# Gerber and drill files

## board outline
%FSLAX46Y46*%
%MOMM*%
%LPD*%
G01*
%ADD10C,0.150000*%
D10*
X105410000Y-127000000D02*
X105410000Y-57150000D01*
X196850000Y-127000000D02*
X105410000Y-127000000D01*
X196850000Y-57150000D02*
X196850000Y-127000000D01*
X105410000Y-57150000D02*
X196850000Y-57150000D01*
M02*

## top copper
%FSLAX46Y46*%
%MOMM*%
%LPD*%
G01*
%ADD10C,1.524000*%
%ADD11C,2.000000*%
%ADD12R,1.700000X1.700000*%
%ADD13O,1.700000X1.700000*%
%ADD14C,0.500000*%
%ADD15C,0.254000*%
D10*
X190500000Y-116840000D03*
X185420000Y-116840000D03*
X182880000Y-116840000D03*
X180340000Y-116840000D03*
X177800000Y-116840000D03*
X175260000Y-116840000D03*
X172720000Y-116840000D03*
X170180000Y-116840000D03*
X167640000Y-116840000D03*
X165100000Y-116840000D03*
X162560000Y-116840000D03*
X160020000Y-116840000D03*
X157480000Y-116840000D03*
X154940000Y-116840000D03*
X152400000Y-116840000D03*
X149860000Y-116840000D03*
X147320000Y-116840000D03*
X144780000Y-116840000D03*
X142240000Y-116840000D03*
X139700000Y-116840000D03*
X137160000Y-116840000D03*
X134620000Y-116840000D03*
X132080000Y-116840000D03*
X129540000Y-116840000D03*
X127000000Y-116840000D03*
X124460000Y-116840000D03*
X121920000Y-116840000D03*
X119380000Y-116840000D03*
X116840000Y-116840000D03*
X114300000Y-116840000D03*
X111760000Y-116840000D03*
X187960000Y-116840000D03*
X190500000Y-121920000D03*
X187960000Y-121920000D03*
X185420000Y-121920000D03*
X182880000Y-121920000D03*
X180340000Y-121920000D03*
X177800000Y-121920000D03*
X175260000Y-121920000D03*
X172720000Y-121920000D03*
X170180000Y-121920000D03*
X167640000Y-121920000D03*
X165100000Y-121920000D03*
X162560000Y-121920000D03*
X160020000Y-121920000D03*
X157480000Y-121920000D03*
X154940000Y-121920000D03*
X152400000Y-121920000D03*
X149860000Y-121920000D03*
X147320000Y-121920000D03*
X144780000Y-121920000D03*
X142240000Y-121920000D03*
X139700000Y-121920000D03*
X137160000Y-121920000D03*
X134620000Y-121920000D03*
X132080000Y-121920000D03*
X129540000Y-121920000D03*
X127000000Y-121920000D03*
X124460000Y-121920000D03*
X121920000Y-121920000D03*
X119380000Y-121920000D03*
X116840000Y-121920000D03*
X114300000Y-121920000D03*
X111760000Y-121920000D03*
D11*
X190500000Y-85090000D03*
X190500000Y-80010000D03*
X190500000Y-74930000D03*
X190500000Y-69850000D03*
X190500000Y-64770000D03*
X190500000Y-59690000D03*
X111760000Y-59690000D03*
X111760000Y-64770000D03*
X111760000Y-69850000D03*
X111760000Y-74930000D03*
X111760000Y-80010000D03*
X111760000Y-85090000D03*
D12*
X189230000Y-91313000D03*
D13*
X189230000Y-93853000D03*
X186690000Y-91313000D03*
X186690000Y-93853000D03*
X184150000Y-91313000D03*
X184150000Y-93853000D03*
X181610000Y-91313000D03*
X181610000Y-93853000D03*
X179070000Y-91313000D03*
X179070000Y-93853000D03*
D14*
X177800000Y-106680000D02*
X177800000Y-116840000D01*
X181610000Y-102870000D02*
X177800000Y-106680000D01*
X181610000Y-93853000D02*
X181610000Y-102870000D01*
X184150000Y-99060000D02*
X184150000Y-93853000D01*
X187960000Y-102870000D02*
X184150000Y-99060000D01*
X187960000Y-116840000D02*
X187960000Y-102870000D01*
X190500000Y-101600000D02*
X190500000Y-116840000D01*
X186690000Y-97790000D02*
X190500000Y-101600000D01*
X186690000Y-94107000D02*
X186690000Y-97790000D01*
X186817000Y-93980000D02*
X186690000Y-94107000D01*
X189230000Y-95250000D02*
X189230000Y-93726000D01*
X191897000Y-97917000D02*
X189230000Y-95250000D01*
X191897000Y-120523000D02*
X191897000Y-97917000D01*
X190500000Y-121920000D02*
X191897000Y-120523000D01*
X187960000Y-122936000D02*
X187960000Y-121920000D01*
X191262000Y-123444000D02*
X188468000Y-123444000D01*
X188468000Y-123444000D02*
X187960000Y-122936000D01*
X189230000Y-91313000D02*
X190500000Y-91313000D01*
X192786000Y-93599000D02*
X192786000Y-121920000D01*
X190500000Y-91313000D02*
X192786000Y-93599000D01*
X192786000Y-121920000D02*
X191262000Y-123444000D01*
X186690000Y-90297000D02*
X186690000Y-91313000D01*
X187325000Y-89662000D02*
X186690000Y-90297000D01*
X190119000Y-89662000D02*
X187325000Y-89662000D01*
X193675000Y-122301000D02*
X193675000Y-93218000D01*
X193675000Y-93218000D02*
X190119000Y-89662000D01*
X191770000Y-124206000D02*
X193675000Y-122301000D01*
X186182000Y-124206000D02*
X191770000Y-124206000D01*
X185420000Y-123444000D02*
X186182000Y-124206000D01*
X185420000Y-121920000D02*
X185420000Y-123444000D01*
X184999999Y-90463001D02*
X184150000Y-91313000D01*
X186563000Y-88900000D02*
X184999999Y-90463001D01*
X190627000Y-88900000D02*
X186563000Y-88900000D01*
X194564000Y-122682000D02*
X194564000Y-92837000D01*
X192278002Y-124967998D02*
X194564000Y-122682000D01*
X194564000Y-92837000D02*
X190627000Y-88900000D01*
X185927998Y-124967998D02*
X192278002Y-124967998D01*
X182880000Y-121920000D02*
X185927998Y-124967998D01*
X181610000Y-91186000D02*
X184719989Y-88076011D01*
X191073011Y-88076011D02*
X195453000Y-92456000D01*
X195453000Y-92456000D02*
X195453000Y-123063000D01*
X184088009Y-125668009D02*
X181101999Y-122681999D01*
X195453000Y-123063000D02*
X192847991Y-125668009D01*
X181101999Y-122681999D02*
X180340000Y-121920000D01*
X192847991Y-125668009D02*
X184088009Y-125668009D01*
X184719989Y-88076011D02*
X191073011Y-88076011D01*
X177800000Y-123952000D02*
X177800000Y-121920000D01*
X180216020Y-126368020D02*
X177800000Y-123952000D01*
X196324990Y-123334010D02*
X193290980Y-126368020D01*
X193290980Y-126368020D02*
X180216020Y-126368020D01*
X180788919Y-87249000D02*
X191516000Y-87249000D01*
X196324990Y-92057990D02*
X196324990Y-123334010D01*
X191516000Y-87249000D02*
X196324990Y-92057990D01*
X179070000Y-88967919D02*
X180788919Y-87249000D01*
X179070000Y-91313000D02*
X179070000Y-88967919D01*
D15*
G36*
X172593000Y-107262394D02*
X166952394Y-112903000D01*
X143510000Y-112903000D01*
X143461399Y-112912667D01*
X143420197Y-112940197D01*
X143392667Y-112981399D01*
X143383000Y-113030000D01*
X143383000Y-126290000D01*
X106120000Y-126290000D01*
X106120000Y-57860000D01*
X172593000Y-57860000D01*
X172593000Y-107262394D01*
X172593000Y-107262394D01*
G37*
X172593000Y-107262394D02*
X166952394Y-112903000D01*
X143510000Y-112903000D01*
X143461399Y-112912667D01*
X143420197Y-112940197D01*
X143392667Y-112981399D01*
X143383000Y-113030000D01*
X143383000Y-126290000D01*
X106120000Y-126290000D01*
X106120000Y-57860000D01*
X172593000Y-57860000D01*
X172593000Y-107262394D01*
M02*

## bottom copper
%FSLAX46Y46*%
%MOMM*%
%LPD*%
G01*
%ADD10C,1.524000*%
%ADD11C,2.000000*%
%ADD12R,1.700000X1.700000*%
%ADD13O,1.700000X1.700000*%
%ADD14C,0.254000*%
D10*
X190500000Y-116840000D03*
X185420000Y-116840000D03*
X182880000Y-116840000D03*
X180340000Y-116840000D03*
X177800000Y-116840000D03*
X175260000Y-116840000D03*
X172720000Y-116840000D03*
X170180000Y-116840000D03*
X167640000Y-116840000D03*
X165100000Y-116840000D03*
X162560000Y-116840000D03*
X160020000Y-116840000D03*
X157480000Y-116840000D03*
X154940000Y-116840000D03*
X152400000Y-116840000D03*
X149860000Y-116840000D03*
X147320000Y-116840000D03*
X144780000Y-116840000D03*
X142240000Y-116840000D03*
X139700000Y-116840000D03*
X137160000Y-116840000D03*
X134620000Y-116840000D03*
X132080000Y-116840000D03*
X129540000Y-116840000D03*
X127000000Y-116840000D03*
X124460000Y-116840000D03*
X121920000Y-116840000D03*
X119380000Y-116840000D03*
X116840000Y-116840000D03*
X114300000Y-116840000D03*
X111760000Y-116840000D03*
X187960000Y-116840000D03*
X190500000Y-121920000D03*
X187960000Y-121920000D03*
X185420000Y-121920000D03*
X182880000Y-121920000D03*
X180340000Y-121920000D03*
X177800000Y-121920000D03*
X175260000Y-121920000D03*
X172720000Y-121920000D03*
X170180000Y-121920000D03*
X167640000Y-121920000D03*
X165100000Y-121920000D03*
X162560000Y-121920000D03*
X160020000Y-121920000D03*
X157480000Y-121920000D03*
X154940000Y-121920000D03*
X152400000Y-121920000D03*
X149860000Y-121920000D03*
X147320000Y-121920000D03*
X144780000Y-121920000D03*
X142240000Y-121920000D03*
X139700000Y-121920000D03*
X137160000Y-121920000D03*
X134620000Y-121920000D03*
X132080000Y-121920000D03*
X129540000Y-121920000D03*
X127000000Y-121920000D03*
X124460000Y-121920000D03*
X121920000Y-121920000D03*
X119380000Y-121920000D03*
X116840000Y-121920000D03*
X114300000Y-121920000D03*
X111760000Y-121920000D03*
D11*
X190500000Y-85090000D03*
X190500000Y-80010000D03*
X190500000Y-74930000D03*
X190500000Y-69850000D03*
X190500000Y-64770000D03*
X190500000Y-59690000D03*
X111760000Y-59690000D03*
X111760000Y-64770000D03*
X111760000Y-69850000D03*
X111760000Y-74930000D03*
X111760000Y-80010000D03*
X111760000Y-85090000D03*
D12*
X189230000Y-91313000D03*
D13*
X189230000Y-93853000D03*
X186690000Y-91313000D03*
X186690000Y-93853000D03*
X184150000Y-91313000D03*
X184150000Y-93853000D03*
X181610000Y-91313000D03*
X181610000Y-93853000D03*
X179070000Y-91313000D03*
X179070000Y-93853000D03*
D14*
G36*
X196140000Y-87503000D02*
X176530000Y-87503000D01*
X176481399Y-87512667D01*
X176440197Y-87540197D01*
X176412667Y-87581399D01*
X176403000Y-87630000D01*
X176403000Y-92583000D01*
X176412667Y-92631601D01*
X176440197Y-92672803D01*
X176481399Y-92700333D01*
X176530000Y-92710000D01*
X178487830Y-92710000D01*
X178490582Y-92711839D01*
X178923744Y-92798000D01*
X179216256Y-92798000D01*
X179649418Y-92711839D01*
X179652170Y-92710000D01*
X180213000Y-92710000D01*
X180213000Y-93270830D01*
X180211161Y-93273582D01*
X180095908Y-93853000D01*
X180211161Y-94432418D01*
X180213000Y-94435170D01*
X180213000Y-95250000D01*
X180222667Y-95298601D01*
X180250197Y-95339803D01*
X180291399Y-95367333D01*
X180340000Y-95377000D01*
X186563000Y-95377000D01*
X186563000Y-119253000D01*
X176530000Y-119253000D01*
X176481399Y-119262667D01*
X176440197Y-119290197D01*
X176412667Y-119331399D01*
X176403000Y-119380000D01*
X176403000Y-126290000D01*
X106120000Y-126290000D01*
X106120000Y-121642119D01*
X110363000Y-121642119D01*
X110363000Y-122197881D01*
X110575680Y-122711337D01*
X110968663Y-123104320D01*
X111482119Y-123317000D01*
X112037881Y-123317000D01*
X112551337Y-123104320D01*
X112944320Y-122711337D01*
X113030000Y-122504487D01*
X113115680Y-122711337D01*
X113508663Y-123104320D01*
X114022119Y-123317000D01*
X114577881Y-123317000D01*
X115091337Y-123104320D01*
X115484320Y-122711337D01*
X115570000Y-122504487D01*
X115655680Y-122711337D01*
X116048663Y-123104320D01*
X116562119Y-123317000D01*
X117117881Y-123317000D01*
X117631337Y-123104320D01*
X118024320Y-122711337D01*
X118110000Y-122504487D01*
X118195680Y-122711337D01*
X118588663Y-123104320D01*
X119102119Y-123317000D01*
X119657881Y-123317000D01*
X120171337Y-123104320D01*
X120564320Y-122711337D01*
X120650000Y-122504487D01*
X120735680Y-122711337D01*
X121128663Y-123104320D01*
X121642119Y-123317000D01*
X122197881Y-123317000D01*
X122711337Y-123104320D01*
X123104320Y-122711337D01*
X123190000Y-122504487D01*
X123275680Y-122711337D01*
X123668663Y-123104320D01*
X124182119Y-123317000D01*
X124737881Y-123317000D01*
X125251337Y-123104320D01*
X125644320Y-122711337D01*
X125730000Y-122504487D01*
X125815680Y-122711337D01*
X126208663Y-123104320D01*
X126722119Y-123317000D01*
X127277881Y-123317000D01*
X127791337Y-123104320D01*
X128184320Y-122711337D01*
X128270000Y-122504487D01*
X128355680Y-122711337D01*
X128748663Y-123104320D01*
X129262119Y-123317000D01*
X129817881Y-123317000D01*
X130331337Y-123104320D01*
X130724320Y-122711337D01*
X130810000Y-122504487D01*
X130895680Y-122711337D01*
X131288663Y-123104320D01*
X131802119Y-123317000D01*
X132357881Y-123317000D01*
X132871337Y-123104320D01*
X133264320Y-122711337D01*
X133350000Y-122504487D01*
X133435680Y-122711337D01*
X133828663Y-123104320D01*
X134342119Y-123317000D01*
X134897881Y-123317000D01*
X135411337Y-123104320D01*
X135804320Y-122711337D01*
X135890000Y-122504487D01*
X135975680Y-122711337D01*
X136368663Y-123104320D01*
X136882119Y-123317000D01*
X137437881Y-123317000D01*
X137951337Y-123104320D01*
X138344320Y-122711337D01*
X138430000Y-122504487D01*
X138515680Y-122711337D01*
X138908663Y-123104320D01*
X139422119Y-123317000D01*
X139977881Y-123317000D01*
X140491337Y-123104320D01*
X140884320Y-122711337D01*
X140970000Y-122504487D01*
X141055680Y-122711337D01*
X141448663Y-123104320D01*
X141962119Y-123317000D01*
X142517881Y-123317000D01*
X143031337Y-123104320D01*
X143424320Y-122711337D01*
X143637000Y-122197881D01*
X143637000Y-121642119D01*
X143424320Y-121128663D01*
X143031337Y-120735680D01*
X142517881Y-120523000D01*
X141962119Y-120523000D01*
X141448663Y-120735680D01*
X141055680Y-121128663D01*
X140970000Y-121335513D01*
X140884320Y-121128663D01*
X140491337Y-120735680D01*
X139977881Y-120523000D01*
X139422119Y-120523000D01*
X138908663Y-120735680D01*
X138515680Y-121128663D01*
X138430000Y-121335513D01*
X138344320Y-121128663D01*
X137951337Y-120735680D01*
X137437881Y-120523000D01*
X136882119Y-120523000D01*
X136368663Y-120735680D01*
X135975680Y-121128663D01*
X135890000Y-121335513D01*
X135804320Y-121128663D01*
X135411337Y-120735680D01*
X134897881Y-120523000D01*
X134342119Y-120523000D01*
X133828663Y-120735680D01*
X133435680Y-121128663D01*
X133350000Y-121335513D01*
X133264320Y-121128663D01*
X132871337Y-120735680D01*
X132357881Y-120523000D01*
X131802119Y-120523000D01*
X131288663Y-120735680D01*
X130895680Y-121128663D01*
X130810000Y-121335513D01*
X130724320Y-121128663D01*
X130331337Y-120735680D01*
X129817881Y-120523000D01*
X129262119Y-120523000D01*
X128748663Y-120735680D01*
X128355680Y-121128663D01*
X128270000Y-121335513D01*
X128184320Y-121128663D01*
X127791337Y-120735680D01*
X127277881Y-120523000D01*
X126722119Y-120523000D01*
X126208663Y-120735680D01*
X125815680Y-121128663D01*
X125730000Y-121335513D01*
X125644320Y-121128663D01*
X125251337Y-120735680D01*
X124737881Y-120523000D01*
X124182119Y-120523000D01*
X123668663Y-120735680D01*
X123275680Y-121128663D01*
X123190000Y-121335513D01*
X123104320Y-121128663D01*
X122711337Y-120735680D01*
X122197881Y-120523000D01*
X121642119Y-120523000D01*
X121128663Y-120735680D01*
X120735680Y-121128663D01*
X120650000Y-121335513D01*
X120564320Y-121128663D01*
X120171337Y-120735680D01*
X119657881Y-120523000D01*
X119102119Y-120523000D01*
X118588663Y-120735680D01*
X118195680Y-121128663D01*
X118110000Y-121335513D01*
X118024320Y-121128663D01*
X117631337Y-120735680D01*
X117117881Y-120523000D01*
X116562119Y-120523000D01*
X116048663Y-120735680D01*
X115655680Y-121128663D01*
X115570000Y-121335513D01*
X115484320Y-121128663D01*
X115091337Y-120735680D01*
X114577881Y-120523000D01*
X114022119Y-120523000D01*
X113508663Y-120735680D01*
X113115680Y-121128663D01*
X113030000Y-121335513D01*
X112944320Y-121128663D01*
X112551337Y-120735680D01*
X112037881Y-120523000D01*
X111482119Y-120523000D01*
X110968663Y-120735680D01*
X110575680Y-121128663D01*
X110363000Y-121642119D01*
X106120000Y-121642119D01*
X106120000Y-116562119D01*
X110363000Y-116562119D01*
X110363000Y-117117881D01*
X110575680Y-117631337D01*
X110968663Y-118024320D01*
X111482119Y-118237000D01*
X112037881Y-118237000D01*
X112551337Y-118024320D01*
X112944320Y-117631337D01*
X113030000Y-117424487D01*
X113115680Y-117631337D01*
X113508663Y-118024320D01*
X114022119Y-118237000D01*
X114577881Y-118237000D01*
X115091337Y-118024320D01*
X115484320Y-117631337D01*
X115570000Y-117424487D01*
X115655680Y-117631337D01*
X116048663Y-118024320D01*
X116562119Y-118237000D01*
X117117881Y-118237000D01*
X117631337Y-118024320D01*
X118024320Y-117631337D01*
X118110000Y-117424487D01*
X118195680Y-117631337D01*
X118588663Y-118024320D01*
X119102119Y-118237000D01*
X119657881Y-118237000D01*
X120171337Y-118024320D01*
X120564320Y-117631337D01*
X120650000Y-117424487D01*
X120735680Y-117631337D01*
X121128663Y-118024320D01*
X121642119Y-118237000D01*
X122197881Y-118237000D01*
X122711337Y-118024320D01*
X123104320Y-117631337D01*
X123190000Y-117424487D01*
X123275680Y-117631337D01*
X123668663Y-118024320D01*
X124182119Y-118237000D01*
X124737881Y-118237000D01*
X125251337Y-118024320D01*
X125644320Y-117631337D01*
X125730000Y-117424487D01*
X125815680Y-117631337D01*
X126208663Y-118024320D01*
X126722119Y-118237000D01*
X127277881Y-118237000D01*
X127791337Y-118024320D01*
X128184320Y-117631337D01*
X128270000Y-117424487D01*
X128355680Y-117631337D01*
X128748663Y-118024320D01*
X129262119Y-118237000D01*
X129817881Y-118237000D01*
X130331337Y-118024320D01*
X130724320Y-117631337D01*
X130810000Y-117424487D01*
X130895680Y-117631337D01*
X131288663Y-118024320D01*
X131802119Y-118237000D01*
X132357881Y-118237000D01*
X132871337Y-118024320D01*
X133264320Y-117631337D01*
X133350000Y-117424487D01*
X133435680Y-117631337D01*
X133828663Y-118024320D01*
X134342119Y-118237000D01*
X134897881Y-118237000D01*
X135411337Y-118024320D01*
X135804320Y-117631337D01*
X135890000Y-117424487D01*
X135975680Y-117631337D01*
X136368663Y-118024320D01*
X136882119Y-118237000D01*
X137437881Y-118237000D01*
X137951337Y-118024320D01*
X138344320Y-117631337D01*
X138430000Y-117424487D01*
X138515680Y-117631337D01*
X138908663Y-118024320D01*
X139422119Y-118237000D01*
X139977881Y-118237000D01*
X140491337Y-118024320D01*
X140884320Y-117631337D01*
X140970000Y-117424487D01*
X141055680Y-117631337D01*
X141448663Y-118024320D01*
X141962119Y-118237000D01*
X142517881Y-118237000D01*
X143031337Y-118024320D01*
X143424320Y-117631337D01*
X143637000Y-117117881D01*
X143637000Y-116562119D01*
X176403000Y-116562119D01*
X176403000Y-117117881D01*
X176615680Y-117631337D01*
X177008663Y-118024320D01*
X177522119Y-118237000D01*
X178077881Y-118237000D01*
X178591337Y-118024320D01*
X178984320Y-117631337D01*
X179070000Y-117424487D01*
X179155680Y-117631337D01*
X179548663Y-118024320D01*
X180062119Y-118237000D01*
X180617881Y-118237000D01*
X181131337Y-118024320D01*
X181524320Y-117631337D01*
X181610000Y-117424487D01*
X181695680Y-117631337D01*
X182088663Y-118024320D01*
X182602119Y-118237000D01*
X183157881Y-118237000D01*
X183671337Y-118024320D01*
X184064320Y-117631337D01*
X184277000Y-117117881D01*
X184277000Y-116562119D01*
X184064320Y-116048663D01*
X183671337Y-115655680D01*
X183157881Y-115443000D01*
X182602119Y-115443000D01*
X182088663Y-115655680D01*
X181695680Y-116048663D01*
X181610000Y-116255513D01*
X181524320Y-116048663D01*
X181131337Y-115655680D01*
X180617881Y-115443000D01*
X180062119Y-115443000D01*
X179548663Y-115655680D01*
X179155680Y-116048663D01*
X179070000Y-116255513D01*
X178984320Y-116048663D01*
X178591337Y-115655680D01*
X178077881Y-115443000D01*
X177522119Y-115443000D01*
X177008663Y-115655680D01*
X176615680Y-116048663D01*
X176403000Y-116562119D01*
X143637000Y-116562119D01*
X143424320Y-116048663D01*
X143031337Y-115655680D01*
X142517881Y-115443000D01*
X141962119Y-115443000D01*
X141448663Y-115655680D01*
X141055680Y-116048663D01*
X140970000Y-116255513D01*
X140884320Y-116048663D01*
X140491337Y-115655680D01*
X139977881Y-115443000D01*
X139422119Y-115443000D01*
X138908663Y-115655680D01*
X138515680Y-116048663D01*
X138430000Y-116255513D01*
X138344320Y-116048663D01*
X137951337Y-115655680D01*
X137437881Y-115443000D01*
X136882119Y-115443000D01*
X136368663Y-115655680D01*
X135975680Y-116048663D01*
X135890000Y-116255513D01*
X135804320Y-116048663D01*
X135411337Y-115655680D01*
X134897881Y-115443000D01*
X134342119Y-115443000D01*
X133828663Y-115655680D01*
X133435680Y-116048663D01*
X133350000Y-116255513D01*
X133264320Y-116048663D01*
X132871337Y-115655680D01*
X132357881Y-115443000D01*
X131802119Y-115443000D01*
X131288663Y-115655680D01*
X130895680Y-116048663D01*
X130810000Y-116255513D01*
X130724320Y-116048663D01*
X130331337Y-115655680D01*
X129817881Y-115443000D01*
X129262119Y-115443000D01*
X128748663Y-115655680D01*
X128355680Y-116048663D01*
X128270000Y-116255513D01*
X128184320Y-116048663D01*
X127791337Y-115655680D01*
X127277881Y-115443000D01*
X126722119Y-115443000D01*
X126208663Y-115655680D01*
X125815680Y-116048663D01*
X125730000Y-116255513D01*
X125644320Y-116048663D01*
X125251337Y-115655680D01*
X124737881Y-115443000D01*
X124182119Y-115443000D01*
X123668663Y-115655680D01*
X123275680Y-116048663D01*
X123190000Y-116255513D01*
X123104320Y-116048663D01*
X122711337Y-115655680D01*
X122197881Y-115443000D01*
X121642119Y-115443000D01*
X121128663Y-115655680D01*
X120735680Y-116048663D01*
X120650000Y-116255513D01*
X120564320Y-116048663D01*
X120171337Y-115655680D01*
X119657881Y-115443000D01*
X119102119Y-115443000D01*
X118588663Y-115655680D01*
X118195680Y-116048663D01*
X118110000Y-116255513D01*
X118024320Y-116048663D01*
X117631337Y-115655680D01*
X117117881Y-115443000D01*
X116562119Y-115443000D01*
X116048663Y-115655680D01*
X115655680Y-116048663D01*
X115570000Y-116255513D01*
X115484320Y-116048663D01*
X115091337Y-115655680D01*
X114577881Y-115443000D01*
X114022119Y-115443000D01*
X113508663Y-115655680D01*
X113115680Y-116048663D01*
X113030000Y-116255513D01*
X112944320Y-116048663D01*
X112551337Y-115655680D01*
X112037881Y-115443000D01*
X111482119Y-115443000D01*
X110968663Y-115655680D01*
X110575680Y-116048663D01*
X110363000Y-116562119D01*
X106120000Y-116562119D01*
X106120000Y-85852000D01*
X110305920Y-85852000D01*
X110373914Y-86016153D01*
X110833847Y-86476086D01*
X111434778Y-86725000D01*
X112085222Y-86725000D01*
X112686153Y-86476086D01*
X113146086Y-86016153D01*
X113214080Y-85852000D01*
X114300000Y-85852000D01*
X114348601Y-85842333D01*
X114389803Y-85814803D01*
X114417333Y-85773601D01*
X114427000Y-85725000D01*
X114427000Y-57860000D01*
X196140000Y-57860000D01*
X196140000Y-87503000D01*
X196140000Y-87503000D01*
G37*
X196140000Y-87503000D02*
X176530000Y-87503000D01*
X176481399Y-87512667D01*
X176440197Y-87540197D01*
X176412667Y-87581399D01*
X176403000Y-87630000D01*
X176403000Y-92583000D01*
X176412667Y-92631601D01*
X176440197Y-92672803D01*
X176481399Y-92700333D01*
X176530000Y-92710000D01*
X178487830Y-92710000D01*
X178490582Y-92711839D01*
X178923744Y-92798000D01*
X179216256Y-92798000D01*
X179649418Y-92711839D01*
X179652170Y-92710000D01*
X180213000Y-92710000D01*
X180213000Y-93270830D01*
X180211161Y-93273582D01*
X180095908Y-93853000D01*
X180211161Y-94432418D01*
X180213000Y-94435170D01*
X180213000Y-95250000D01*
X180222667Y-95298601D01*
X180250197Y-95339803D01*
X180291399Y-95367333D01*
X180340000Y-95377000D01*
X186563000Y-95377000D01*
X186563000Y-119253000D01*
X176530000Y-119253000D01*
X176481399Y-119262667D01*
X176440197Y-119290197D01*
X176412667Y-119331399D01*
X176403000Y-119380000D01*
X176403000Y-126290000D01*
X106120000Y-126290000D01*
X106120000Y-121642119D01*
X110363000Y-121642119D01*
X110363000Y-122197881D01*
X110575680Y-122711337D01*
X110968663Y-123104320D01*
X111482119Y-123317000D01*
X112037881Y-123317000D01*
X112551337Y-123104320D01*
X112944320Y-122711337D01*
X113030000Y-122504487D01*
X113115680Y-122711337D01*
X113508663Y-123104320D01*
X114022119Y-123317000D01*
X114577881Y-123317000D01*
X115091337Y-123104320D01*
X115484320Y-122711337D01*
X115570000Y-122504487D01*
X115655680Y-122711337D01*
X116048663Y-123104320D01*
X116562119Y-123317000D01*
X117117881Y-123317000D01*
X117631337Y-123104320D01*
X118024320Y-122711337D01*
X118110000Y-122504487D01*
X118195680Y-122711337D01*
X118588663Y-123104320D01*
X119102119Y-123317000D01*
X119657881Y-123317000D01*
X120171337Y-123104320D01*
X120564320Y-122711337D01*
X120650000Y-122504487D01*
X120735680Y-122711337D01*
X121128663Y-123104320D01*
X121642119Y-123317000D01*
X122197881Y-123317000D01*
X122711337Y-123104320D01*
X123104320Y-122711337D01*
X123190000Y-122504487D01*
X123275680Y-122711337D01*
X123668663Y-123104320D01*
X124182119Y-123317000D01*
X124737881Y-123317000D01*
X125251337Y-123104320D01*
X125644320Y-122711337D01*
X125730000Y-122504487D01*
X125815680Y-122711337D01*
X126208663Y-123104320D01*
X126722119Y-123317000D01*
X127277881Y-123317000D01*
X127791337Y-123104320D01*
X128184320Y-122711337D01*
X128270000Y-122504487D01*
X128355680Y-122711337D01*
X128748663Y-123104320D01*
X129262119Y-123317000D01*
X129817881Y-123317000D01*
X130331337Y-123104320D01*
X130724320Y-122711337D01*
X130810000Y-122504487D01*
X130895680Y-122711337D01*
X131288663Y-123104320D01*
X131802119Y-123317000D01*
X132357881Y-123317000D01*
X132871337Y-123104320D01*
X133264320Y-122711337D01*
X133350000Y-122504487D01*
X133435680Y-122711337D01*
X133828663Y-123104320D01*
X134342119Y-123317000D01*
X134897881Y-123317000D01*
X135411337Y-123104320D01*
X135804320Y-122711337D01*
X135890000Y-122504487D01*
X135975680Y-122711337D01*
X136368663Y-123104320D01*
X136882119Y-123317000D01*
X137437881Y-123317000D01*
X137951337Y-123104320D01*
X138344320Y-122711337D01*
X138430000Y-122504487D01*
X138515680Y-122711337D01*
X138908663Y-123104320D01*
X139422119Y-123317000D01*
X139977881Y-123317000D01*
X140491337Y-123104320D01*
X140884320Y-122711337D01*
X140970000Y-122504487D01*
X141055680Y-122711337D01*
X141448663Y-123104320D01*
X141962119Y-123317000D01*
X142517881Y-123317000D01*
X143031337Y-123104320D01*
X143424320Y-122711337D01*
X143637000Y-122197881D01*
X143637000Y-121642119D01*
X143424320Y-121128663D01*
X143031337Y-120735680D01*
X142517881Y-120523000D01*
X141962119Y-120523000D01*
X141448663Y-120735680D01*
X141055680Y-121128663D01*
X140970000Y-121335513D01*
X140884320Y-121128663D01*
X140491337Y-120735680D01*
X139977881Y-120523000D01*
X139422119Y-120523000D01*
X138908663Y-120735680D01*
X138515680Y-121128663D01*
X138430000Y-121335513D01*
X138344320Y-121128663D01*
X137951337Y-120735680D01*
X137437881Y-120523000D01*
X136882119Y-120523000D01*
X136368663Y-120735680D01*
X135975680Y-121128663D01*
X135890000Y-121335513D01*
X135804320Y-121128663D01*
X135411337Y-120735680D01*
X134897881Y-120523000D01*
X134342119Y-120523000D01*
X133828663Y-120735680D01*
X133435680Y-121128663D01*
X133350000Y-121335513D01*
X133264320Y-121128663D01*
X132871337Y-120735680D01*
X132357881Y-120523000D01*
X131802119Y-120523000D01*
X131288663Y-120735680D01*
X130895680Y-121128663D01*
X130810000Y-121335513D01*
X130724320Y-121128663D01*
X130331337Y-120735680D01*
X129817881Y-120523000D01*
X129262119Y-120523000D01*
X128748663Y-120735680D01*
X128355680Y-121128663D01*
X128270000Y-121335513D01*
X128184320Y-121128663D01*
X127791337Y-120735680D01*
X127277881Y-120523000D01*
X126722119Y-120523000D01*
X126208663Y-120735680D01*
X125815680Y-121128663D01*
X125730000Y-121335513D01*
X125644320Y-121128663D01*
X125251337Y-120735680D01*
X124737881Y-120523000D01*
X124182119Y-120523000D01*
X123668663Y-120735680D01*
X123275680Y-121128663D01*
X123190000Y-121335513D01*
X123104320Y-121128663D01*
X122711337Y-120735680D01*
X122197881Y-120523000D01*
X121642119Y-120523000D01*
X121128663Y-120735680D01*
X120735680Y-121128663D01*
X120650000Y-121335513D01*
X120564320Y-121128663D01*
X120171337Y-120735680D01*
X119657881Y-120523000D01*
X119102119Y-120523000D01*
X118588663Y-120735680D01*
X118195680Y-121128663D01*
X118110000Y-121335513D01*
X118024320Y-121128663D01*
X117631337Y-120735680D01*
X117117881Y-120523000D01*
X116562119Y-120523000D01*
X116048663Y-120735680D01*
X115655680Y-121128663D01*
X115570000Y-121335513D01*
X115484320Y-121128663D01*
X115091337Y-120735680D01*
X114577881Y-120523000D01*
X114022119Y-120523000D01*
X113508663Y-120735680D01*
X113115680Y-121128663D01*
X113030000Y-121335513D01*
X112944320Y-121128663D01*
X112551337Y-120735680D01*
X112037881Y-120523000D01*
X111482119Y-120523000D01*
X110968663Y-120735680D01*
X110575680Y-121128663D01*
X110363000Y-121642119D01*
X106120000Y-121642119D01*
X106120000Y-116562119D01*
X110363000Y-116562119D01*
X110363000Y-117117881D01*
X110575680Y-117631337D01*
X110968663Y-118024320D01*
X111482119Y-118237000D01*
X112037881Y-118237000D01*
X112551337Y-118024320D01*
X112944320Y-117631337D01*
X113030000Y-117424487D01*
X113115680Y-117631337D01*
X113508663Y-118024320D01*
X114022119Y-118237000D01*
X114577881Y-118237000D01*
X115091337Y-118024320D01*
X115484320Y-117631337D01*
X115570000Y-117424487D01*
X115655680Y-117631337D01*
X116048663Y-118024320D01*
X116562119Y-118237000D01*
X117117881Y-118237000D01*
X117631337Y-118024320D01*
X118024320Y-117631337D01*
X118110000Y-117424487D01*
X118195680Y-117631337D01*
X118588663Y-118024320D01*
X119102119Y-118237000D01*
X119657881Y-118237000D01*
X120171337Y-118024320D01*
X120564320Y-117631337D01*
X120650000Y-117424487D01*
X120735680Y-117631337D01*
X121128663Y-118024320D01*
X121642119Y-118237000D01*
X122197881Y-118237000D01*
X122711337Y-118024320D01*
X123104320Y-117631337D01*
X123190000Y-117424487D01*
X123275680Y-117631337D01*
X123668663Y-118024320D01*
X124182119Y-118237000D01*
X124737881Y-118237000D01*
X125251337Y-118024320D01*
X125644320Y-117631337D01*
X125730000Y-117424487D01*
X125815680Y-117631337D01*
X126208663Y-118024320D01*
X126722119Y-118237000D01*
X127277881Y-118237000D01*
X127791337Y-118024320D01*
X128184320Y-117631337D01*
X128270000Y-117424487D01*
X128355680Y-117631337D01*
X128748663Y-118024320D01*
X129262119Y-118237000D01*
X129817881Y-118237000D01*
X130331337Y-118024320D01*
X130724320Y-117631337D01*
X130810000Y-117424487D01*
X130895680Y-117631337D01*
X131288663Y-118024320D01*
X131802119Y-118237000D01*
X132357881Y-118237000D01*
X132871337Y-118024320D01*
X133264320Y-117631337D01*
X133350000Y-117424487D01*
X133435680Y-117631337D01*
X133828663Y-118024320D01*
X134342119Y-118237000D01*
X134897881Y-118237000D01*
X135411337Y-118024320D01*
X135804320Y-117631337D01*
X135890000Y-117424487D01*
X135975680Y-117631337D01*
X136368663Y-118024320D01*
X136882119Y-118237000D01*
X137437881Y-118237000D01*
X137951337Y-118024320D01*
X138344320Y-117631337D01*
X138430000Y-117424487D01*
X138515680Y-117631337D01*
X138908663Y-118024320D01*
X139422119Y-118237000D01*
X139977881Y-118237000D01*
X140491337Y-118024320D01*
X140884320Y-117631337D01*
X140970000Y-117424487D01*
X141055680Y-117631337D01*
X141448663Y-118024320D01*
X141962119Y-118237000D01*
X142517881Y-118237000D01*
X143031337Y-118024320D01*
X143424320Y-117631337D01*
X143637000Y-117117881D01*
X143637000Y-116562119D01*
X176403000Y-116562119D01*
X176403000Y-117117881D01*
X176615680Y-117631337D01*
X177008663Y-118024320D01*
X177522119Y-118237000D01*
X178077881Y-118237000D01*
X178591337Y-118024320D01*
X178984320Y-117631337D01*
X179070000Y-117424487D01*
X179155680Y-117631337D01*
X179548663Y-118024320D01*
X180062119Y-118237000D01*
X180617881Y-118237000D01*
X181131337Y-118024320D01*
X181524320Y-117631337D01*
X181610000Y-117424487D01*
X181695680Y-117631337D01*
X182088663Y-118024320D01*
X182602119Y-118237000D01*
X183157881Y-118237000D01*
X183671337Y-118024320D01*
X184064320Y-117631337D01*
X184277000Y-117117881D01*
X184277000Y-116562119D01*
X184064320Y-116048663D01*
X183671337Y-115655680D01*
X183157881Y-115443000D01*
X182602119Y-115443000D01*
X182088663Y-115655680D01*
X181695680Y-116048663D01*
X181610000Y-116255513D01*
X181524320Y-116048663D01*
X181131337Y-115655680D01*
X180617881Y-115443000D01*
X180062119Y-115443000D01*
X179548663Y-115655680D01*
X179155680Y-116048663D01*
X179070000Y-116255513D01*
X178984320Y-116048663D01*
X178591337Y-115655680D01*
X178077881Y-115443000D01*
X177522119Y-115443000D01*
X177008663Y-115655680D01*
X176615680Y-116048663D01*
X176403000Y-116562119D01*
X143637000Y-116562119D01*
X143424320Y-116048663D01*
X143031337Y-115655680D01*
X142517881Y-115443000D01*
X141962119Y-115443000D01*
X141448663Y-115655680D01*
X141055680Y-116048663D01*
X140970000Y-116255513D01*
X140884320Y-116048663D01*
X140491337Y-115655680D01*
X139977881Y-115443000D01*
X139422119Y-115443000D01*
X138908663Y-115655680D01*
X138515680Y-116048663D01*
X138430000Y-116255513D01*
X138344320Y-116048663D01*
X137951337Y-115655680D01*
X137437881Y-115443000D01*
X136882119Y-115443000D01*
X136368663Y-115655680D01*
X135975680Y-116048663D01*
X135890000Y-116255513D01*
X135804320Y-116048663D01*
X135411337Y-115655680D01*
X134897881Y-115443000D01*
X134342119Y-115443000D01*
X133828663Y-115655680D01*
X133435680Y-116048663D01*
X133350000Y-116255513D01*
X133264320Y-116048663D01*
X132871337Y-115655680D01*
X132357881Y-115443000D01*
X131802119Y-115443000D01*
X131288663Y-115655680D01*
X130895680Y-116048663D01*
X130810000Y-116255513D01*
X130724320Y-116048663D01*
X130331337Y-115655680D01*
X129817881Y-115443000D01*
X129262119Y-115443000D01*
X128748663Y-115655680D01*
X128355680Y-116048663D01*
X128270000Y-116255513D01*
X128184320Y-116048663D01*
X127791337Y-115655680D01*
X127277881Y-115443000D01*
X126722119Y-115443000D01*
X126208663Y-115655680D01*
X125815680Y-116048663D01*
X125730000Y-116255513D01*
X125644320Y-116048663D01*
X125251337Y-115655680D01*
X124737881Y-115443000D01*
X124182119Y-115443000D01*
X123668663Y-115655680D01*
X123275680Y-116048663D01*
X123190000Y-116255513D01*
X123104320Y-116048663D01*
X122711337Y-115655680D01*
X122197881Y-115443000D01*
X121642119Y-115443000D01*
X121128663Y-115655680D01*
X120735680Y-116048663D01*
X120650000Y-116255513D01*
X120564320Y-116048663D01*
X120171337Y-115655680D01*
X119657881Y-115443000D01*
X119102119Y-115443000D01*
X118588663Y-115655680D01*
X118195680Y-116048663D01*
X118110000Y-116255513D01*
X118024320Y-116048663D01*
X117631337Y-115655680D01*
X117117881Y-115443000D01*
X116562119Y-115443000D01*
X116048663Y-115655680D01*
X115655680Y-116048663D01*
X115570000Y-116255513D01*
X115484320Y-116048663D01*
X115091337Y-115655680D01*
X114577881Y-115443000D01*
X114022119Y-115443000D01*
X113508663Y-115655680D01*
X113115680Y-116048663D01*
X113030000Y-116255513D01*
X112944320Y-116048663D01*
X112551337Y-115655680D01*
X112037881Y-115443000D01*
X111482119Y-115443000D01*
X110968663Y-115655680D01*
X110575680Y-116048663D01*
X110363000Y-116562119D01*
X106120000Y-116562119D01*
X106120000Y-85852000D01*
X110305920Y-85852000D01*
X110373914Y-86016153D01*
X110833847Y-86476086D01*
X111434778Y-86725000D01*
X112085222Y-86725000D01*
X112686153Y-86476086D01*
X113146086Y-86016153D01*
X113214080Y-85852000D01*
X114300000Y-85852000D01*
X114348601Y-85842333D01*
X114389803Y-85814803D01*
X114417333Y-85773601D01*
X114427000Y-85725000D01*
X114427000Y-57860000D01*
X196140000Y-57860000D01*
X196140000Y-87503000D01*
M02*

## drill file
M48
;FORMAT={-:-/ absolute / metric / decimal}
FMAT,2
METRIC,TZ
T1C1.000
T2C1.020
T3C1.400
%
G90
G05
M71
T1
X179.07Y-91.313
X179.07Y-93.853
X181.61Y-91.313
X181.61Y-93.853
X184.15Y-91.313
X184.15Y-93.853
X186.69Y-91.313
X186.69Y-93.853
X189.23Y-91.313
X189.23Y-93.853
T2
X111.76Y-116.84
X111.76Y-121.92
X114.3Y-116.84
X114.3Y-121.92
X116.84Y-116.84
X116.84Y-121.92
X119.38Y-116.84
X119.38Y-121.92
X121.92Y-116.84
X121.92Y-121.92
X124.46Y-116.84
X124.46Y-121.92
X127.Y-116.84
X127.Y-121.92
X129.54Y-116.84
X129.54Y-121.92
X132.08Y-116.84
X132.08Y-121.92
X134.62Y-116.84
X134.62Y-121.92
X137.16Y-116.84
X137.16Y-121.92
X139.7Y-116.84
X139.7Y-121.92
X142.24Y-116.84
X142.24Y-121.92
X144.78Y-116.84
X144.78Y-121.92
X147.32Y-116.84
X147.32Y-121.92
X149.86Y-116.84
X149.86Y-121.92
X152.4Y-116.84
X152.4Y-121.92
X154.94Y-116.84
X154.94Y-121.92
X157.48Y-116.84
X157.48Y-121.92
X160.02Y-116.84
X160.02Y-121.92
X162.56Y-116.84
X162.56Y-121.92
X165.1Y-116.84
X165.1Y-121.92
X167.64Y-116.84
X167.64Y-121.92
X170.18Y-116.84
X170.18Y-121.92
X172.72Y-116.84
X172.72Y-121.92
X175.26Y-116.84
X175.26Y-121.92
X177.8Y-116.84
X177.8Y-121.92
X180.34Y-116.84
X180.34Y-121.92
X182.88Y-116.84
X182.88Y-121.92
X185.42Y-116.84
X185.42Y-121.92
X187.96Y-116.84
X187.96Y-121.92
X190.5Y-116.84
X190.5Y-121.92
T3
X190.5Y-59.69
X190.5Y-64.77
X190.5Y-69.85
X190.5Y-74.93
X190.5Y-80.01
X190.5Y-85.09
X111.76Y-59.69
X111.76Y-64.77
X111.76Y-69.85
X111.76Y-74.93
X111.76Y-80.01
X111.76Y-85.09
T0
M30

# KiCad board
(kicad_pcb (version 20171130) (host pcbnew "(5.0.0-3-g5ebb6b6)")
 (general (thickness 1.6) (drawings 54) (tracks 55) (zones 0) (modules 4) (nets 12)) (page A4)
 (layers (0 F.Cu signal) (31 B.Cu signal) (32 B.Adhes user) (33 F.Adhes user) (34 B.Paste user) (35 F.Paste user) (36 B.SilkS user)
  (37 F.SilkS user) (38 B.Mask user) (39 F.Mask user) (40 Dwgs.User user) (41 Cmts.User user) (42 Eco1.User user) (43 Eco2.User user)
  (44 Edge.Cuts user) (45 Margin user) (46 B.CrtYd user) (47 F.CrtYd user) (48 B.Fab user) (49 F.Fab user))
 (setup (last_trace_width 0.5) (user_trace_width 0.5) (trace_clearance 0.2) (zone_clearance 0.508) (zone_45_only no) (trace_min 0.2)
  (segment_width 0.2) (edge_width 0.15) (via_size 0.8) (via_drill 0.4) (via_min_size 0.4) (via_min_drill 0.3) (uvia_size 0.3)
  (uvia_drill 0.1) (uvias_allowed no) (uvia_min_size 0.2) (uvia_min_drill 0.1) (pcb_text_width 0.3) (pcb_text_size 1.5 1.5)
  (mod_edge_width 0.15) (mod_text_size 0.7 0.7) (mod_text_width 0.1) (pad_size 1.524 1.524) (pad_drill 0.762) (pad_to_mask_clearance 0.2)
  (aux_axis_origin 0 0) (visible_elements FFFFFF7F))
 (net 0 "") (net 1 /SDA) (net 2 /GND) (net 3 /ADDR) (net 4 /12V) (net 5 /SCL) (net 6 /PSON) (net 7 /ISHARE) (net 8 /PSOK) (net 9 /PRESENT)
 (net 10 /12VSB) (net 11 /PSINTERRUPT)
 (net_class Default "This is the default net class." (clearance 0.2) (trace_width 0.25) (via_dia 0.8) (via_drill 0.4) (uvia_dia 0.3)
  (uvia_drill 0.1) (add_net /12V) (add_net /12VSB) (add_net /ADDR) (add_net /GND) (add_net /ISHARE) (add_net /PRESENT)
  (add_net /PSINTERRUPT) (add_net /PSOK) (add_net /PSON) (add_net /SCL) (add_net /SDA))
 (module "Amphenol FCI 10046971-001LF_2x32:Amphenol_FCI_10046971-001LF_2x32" (layer B.Cu) (at 151.13 119.38 270)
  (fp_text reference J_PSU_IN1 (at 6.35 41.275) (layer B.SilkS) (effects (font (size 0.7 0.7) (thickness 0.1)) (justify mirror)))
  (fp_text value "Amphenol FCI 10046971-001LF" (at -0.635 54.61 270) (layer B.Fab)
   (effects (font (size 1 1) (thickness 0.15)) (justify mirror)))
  (pad 32 thru_hole circle (at -2.54 -39.37 270) (size 1.524 1.524) (drill 1.02) (layers *.Cu *.Mask) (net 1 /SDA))
  (pad 30 thru_hole circle (at -2.54 -34.29 270) (size 1.524 1.524) (drill 1.02) (layers *.Cu *.Mask) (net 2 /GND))
  (pad 29 thru_hole circle (at -2.54 -31.75 270) (size 1.524 1.524) (drill 1.02) (layers *.Cu *.Mask))
  (pad 28 thru_hole circle (at -2.54 -29.21 270) (size 1.524 1.524) (drill 1.02) (layers *.Cu *.Mask))
  (pad 27 thru_hole circle (at -2.54 -26.67 270) (size 1.524 1.524) (drill 1.02) (layers *.Cu *.Mask) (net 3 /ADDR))
  (pad 26 thru_hole circle (at -2.54 -24.13 270) (size 1.524 1.524) (drill 1.02) (layers *.Cu *.Mask) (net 2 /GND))
  (pad 25 thru_hole circle (at -2.54 -21.59 270) (size 1.524 1.524) (drill 1.02) (layers *.Cu *.Mask) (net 2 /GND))
  (pad 24 thru_hole circle (at -2.54 -19.05 270) (size 1.524 1.524) (drill 1.02) (layers *.Cu *.Mask) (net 2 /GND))
  (pad 23 thru_hole circle (at -2.54 -16.51 270) (size 1.524 1.524) (drill 1.02) (layers *.Cu *.Mask) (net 2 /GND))
  (pad 22 thru_hole circle (at -2.54 -13.97 270) (size 1.524 1.524) (drill 1.02) (layers *.Cu *.Mask) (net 2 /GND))
  (pad 21 thru_hole circle (at -2.54 -11.43 270) (size 1.524 1.524) (drill 1.02) (layers *.Cu *.Mask) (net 2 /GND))
  (pad 20 thru_hole circle (at -2.54 -8.89 270) (size 1.524 1.524) (drill 1.02) (layers *.Cu *.Mask) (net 2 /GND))
  (pad 19 thru_hole circle (at -2.54 -6.35 270) (size 1.524 1.524) (drill 1.02) (layers *.Cu *.Mask) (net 2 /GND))
  (pad 18 thru_hole circle (at -2.54 -3.81 270) (size 1.524 1.524) (drill 1.02) (layers *.Cu *.Mask) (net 2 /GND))
  (pad 17 thru_hole circle (at -2.54 -1.27 270) (size 1.524 1.524) (drill 1.02) (layers *.Cu *.Mask) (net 2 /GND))
  (pad 16 thru_hole circle (at -2.54 1.27 270) (size 1.524 1.524) (drill 1.02) (layers *.Cu *.Mask) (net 2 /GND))
  (pad 15 thru_hole circle (at -2.54 3.81 270) (size 1.524 1.524) (drill 1.02) (layers *.Cu *.Mask) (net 2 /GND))
  (pad 14 thru_hole circle (at -2.54 6.35 270) (size 1.524 1.524) (drill 1.02) (layers *.Cu *.Mask) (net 2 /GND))
  (pad 13 thru_hole circle (at -2.54 8.89 270) (size 1.524 1.524) (drill 1.02) (layers *.Cu *.Mask) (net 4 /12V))
  (pad 12 thru_hole circle (at -2.54 11.43 270) (size 1.524 1.524) (drill 1.02) (layers *.Cu *.Mask) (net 4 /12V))
  (pad 11 thru_hole circle (at -2.54 13.97 270) (size 1.524 1.524) (drill 1.02) (layers *.Cu *.Mask) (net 4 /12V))
  (pad 10 thru_hole circle (at -2.54 16.51 270) (size 1.524 1.524) (drill 1.02) (layers *.Cu *.Mask) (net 4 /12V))
  (pad 9 thru_hole circle (at -2.54 19.05 270) (size 1.524 1.524) (drill 1.02) (layers *.Cu *.Mask) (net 4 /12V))
  (pad 8 thru_hole circle (at -2.54 21.59 270) (size 1.524 1.524) (drill 1.02) (layers *.Cu *.Mask) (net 4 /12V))
  (pad 7 thru_hole circle (at -2.54 24.13 270) (size 1.524 1.524) (drill 1.02) (layers *.Cu *.Mask) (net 4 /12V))
  (pad 6 thru_hole circle (at -2.54 26.67 270) (size 1.524 1.524) (drill 1.02) (layers *.Cu *.Mask) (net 4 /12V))
  (pad 5 thru_hole circle (at -2.54 29.21 270) (size 1.524 1.524) (drill 1.02) (layers *.Cu *.Mask) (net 4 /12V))
  (pad 4 thru_hole circle (at -2.54 31.75 270) (size 1.524 1.524) (drill 1.02) (layers *.Cu *.Mask) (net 4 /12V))
  (pad 3 thru_hole circle (at -2.54 34.29 270) (size 1.524 1.524) (drill 1.02) (layers *.Cu *.Mask) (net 4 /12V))
  (pad 2 thru_hole circle (at -2.54 36.83 270) (size 1.524 1.524) (drill 1.02) (layers *.Cu *.Mask) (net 4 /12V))
  (pad 1 thru_hole circle (at -2.54 39.37 270) (size 1.524 1.524) (drill 1.02) (layers *.Cu *.Mask) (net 4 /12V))
  (pad 31 thru_hole circle (at -2.54 -36.83 270) (size 1.524 1.524) (drill 1.02) (layers *.Cu *.Mask) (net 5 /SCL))
  (pad 33 thru_hole circle (at 2.54 -39.37 270) (size 1.524 1.524) (drill 1.02) (layers *.Cu *.Mask) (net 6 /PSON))
  (pad 34 thru_hole circle (at 2.54 -36.83 270) (size 1.524 1.524) (drill 1.02) (layers *.Cu *.Mask) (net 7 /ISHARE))
  (pad 35 thru_hole circle (at 2.54 -34.29 270) (size 1.524 1.524) (drill 1.02) (layers *.Cu *.Mask) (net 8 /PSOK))
  (pad 36 thru_hole circle (at 2.54 -31.75 270) (size 1.524 1.524) (drill 1.02) (layers *.Cu *.Mask) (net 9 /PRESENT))
  (pad 37 thru_hole circle (at 2.54 -29.21 270) (size 1.524 1.524) (drill 1.02) (layers *.Cu *.Mask) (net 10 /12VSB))
  (pad 38 thru_hole circle (at 2.54 -26.67 270) (size 1.524 1.524) (drill 1.02) (layers *.Cu *.Mask) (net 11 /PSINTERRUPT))
  (pad 39 thru_hole circle (at 2.54 -24.13 270) (size 1.524 1.524) (drill 1.02) (layers *.Cu *.Mask) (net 2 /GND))
  (pad 40 thru_hole circle (at 2.54 -21.59 270) (size 1.524 1.524) (drill 1.02) (layers *.Cu *.Mask) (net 2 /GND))
  (pad 41 thru_hole circle (at 2.54 -19.05 270) (size 1.524 1.524) (drill 1.02) (layers *.Cu *.Mask) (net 2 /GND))
  (pad 42 thru_hole circle (at 2.54 -16.51 270) (size 1.524 1.524) (drill 1.02) (layers *.Cu *.Mask) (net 2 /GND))
  (pad 43 thru_hole circle (at 2.54 -13.97 270) (size 1.524 1.524) (drill 1.02) (layers *.Cu *.Mask) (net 2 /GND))
  (pad 44 thru_hole circle (at 2.54 -11.43 270) (size 1.524 1.524) (drill 1.02) (layers *.Cu *.Mask) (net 2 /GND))
  (pad 45 thru_hole circle (at 2.54 -8.89 270) (size 1.524 1.524) (drill 1.02) (layers *.Cu *.Mask) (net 2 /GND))
  (pad 46 thru_hole circle (at 2.54 -6.35 270) (size 1.524 1.524) (drill 1.02) (layers *.Cu *.Mask) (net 2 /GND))
  (pad 47 thru_hole circle (at 2.54 -3.81 270) (size 1.524 1.524) (drill 1.02) (layers *.Cu *.Mask) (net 2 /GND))
  (pad 48 thru_hole circle (at 2.54 -1.27 270) (size 1.524 1.524) (drill 1.02) (layers *.Cu *.Mask) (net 2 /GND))
  (pad 49 thru_hole circle (at 2.54 1.27 270) (size 1.524 1.524) (drill 1.02) (layers *.Cu *.Mask) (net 2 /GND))
  (pad 50 thru_hole circle (at 2.54 3.81 270) (size 1.524 1.524) (drill 1.02) (layers *.Cu *.Mask) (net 2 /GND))
  (pad 51 thru_hole circle (at 2.54 6.35 270) (size 1.524 1.524) (drill 1.02) (layers *.Cu *.Mask) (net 2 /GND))
  (pad 52 thru_hole circle (at 2.54 8.89 270) (size 1.524 1.524) (drill 1.02) (layers *.Cu *.Mask) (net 4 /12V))
  (pad 53 thru_hole circle (at 2.54 11.43 270) (size 1.524 1.524) (drill 1.02) (layers *.Cu *.Mask) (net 4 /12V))
  (pad 54 thru_hole circle (at 2.54 13.97 270) (size 1.524 1.524) (drill 1.02) (layers *.Cu *.Mask) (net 4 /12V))
  (pad 55 thru_hole circle (at 2.54 16.51 270) (size 1.524 1.524) (drill 1.02) (layers *.Cu *.Mask) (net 4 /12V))
  (pad 56 thru_hole circle (at 2.54 19.05 270) (size 1.524 1.524) (drill 1.02) (layers *.Cu *.Mask) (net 4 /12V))
  (pad 57 thru_hole circle (at 2.54 21.59 270) (size 1.524 1.524) (drill 1.02) (layers *.Cu *.Mask) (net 4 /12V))
  (pad 58 thru_hole circle (at 2.54 24.13 270) (size 1.524 1.524) (drill 1.02) (layers *.Cu *.Mask) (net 4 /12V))
  (pad 59 thru_hole circle (at 2.54 26.67 270) (size 1.524 1.524) (drill 1.02) (layers *.Cu *.Mask) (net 4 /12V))
  (pad 60 thru_hole circle (at 2.54 29.21 270) (size 1.524 1.524) (drill 1.02) (layers *.Cu *.Mask) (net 4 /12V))
  (pad 61 thru_hole circle (at 2.54 31.75 270) (size 1.524 1.524) (drill 1.02) (layers *.Cu *.Mask) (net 4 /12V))
  (pad 62 thru_hole circle (at 2.54 34.29 270) (size 1.524 1.524) (drill 1.02) (layers *.Cu *.Mask) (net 4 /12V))
  (pad 63 thru_hole circle (at 2.54 36.83 270) (size 1.524 1.524) (drill 1.02) (layers *.Cu *.Mask) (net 4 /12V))
  (pad 64 thru_hole circle (at 2.54 39.37 270) (size 1.524 1.524) (drill 1.02) (layers *.Cu *.Mask) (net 4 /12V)))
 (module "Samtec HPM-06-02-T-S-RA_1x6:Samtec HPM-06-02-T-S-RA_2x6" (layer F.Cu) (at 190.5 72.39)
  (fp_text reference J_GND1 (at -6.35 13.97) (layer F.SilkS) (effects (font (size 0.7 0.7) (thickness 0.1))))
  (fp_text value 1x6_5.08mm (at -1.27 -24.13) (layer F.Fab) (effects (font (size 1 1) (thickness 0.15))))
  (pad 6 thru_hole circle (at 0 12.7) (size 2 2) (drill 1.4) (layers *.Cu *.Mask) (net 2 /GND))
  (pad 5 thru_hole circle (at 0 7.62) (size 2 2) (drill 1.4) (layers *.Cu *.Mask) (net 2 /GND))
  (pad 4 thru_hole circle (at 0 2.54) (size 2 2) (drill 1.4) (layers *.Cu *.Mask) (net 2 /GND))
  (pad 3 thru_hole circle (at 0 -2.54) (size 2 2) (drill 1.4) (layers *.Cu *.Mask) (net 2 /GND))
  (pad 2 thru_hole circle (at 0 -7.62) (size 2 2) (drill 1.4) (layers *.Cu *.Mask) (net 2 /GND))
  (pad 1 thru_hole circle (at 0 -12.7) (size 2 2) (drill 1.4) (layers *.Cu *.Mask) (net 2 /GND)))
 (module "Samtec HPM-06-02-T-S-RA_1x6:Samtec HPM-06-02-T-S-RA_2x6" (layer F.Cu) (at 111.76 72.39)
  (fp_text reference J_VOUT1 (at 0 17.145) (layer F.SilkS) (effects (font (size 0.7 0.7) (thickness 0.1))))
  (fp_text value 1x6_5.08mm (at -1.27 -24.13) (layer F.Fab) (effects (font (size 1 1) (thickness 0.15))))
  (pad 1 thru_hole circle (at 0 -12.7) (size 2 2) (drill 1.4) (layers *.Cu *.Mask) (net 4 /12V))
  (pad 2 thru_hole circle (at 0 -7.62) (size 2 2) (drill 1.4) (layers *.Cu *.Mask) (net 4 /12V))
  (pad 3 thru_hole circle (at 0 -2.54) (size 2 2) (drill 1.4) (layers *.Cu *.Mask) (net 4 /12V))
  (pad 4 thru_hole circle (at 0 2.54) (size 2 2) (drill 1.4) (layers *.Cu *.Mask) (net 4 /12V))
  (pad 5 thru_hole circle (at 0 7.62) (size 2 2) (drill 1.4) (layers *.Cu *.Mask) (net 4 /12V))
  (pad 6 thru_hole circle (at 0 12.7) (size 2 2) (drill 1.4) (layers *.Cu *.Mask) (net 4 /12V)))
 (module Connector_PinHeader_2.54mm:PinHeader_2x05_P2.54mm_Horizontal (layer F.Cu) (at 189.23 91.313 270)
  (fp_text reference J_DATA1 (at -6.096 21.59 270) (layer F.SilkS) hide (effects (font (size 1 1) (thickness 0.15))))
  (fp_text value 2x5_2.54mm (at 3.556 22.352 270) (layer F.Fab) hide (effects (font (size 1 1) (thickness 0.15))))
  (pad 1 thru_hole rect (at 0 0 270) (size 1.7 1.7) (drill 1) (layers *.Cu *.Mask) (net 7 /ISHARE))
  (pad 2 thru_hole oval (at 2.54 0 270) (size 1.7 1.7) (drill 1) (layers *.Cu *.Mask) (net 6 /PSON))
  (pad 3 thru_hole oval (at 0 2.54 270) (size 1.7 1.7) (drill 1) (layers *.Cu *.Mask) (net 8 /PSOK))
  (pad 4 thru_hole oval (at 2.54 2.54 270) (size 1.7 1.7) (drill 1) (layers *.Cu *.Mask) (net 1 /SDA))
  (pad 5 thru_hole oval (at 0 5.08 270) (size 1.7 1.7) (drill 1) (layers *.Cu *.Mask) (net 9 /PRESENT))
  (pad 6 thru_hole oval (at 2.54 5.08 270) (size 1.7 1.7) (drill 1) (layers *.Cu *.Mask) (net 5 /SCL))
  (pad 7 thru_hole oval (at 0 7.62 270) (size 1.7 1.7) (drill 1) (layers *.Cu *.Mask) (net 10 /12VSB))
  (pad 8 thru_hole oval (at 2.54 7.62 270) (size 1.7 1.7) (drill 1) (layers *.Cu *.Mask) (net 3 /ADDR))
  (pad 9 thru_hole oval (at 0 10.16 270) (size 1.7 1.7) (drill 1) (layers *.Cu *.Mask) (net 11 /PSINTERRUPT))
  (pad 10 thru_hole oval (at 2.54 10.16 270) (size 1.7 1.7) (drill 1) (layers *.Cu *.Mask) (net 2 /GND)))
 (gr_line (start 105.41 127) (end 105.41 57.15) (layer Edge.Cuts) (width 0.15))
 (gr_line (start 196.85 127) (end 105.41 127) (layer Edge.Cuts) (width 0.15))
 (gr_line (start 196.85 57.15) (end 196.85 127) (layer Edge.Cuts) (width 0.15))
 (gr_line (start 105.41 57.15) (end 196.85 57.15) (layer Edge.Cuts) (width 0.15))
 (segment (start 177.8 106.68) (end 177.8 116.84) (width 0.5) (layer F.Cu) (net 3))
 (segment (start 181.61 102.87) (end 177.8 106.68) (width 0.5) (layer F.Cu) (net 3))
 (segment (start 181.61 93.853) (end 181.61 102.87) (width 0.5) (layer F.Cu) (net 3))
 (segment (start 184.15 99.06) (end 184.15 93.853) (width 0.5) (layer F.Cu) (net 5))
 (segment (start 187.96 102.87) (end 184.15 99.06) (width 0.5) (layer F.Cu) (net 5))
 (segment (start 187.96 116.84) (end 187.96 102.87) (width 0.5) (layer F.Cu) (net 5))
 (segment (start 190.5 101.6) (end 190.5 116.84) (width 0.5) (layer F.Cu) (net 1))
 (segment (start 186.69 97.79) (end 190.5 101.6) (width 0.5) (layer F.Cu) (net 1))
 (segment (start 186.69 94.107) (end 186.69 97.79) (width 0.5) (layer F.Cu) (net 1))
 (segment (start 186.817 93.98) (end 186.69 94.107) (width 0.5) (layer F.Cu) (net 1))
 (segment (start 189.23 95.25) (end 189.23 93.726) (width 0.5) (layer F.Cu) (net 6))
 (segment (start 191.897 97.917) (end 189.23 95.25) (width 0.5) (layer F.Cu) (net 6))
 (segment (start 191.897 120.523) (end 191.897 97.917) (width 0.5) (layer F.Cu) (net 6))
 (segment (start 190.5 121.92) (end 191.897 120.523) (width 0.5) (layer F.Cu) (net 6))
 (segment (start 187.96 122.936) (end 187.96 121.92) (width 0.5) (layer F.Cu) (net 7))
 (segment (start 191.262 123.444) (end 188.468 123.444) (width 0.5) (layer F.Cu) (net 7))
 (segment (start 188.468 123.444) (end 187.96 122.936) (width 0.5) (layer F.Cu) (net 7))
 (segment (start 189.23 91.313) (end 190.5 91.313) (width 0.5) (layer F.Cu) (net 7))
 (segment (start 192.786 93.599) (end 192.786 121.92) (width 0.5) (layer F.Cu) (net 7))
 (segment (start 190.5 91.313) (end 192.786 93.599) (width 0.5) (layer F.Cu) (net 7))
 (segment (start 192.786 121.92) (end 191.262 123.444) (width 0.5) (layer F.Cu) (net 7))
 (segment (start 186.69 90.297) (end 186.69 91.313) (width 0.5) (layer F.Cu) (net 8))
 (segment (start 187.325 89.662) (end 186.69 90.297) (width 0.5) (layer F.Cu) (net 8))
 (segment (start 190.119 89.662) (end 187.325 89.662) (width 0.5) (layer F.Cu) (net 8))
 (segment (start 193.675 122.301) (end 193.675 93.218) (width 0.5) (layer F.Cu) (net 8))
 (segment (start 193.675 93.218) (end 190.119 89.662) (width 0.5) (layer F.Cu) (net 8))
 (segment (start 191.77 124.206) (end 193.675 122.301) (width 0.5) (layer F.Cu) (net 8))
 (segment (start 186.182 124.206) (end 191.77 124.206) (width 0.5) (layer F.Cu) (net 8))
 (segment (start 185.42 123.444) (end 186.182 124.206) (width 0.5) (layer F.Cu) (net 8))
 (segment (start 185.42 121.92) (end 185.42 123.444) (width 0.5) (layer F.Cu) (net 8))
 (segment (start 184.999999 90.463001) (end 184.15 91.313) (width 0.5) (layer F.Cu) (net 9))
 (segment (start 186.563 88.9) (end 184.999999 90.463001) (width 0.5) (layer F.Cu) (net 9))
 (segment (start 190.627 88.9) (end 186.563 88.9) (width 0.5) (layer F.Cu) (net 9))
 (segment (start 194.564 122.682) (end 194.564 92.837) (width 0.5) (layer F.Cu) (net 9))
 (segment (start 192.278002 124.967998) (end 194.564 122.682) (width 0.5) (layer F.Cu) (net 9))
 (segment (start 194.564 92.837) (end 190.627 88.9) (width 0.5) (layer F.Cu) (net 9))
 (segment (start 185.927998 124.967998) (end 192.278002 124.967998) (width 0.5) (layer F.Cu) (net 9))
 (segment (start 182.88 121.92) (end 185.927998 124.967998) (width 0.5) (layer F.Cu) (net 9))
 (segment (start 181.61 91.186) (end 184.719989 88.076011) (width 0.5) (layer F.Cu) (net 10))
 (segment (start 191.073011 88.076011) (end 195.453 92.456) (width 0.5) (layer F.Cu) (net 10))
 (segment (start 195.453 92.456) (end 195.453 123.063) (width 0.5) (layer F.Cu) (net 10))
 (segment (start 184.088009 125.668009) (end 181.101999 122.681999) (width 0.5) (layer F.Cu) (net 10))
 (segment (start 195.453 123.063) (end 192.847991 125.668009) (width 0.5) (layer F.Cu) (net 10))
 (segment (start 181.101999 122.681999) (end 180.34 121.92) (width 0.5) (layer F.Cu) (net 10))
 (segment (start 192.847991 125.668009) (end 184.088009 125.668009) (width 0.5) (layer F.Cu) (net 10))
 (segment (start 184.719989 88.076011) (end 191.073011 88.076011) (width 0.5) (layer F.Cu) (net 10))
 (segment (start 177.8 123.952) (end 177.8 121.92) (width 0.5) (layer F.Cu) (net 11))
 (segment (start 180.21602 126.36802) (end 177.8 123.952) (width 0.5) (layer F.Cu) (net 11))
 (segment (start 196.32499 123.33401) (end 193.29098 126.36802) (width 0.5) (layer F.Cu) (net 11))
 (segment (start 193.29098 126.36802) (end 180.21602 126.36802) (width 0.5) (layer F.Cu) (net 11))
 (segment (start 180.788919 87.249) (end 191.516 87.249) (width 0.5) (layer F.Cu) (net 11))
 (segment (start 196.32499 92.05799) (end 196.32499 123.33401) (width 0.5) (layer F.Cu) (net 11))
 (segment (start 191.516 87.249) (end 196.32499 92.05799) (width 0.5) (layer F.Cu) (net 11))
 (segment (start 179.07 88.967919) (end 180.788919 87.249) (width 0.5) (layer F.Cu) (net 11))
 (segment (start 179.07 91.313) (end 179.07 88.967919) (width 0.5) (layer F.Cu) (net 11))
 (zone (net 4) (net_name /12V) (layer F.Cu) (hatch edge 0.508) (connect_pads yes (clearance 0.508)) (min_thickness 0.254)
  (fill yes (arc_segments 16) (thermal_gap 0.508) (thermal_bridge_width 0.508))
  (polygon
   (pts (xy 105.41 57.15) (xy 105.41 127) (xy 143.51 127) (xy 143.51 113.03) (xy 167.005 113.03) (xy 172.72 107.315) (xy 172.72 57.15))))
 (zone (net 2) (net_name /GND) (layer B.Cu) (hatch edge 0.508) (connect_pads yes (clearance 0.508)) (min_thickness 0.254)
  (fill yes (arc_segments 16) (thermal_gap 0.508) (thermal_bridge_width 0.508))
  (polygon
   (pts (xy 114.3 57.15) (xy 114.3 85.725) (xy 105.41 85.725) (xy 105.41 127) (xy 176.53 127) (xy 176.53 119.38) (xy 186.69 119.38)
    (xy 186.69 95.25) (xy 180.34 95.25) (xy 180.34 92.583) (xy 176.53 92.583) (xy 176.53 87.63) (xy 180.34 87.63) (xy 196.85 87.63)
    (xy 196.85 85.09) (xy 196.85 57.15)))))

